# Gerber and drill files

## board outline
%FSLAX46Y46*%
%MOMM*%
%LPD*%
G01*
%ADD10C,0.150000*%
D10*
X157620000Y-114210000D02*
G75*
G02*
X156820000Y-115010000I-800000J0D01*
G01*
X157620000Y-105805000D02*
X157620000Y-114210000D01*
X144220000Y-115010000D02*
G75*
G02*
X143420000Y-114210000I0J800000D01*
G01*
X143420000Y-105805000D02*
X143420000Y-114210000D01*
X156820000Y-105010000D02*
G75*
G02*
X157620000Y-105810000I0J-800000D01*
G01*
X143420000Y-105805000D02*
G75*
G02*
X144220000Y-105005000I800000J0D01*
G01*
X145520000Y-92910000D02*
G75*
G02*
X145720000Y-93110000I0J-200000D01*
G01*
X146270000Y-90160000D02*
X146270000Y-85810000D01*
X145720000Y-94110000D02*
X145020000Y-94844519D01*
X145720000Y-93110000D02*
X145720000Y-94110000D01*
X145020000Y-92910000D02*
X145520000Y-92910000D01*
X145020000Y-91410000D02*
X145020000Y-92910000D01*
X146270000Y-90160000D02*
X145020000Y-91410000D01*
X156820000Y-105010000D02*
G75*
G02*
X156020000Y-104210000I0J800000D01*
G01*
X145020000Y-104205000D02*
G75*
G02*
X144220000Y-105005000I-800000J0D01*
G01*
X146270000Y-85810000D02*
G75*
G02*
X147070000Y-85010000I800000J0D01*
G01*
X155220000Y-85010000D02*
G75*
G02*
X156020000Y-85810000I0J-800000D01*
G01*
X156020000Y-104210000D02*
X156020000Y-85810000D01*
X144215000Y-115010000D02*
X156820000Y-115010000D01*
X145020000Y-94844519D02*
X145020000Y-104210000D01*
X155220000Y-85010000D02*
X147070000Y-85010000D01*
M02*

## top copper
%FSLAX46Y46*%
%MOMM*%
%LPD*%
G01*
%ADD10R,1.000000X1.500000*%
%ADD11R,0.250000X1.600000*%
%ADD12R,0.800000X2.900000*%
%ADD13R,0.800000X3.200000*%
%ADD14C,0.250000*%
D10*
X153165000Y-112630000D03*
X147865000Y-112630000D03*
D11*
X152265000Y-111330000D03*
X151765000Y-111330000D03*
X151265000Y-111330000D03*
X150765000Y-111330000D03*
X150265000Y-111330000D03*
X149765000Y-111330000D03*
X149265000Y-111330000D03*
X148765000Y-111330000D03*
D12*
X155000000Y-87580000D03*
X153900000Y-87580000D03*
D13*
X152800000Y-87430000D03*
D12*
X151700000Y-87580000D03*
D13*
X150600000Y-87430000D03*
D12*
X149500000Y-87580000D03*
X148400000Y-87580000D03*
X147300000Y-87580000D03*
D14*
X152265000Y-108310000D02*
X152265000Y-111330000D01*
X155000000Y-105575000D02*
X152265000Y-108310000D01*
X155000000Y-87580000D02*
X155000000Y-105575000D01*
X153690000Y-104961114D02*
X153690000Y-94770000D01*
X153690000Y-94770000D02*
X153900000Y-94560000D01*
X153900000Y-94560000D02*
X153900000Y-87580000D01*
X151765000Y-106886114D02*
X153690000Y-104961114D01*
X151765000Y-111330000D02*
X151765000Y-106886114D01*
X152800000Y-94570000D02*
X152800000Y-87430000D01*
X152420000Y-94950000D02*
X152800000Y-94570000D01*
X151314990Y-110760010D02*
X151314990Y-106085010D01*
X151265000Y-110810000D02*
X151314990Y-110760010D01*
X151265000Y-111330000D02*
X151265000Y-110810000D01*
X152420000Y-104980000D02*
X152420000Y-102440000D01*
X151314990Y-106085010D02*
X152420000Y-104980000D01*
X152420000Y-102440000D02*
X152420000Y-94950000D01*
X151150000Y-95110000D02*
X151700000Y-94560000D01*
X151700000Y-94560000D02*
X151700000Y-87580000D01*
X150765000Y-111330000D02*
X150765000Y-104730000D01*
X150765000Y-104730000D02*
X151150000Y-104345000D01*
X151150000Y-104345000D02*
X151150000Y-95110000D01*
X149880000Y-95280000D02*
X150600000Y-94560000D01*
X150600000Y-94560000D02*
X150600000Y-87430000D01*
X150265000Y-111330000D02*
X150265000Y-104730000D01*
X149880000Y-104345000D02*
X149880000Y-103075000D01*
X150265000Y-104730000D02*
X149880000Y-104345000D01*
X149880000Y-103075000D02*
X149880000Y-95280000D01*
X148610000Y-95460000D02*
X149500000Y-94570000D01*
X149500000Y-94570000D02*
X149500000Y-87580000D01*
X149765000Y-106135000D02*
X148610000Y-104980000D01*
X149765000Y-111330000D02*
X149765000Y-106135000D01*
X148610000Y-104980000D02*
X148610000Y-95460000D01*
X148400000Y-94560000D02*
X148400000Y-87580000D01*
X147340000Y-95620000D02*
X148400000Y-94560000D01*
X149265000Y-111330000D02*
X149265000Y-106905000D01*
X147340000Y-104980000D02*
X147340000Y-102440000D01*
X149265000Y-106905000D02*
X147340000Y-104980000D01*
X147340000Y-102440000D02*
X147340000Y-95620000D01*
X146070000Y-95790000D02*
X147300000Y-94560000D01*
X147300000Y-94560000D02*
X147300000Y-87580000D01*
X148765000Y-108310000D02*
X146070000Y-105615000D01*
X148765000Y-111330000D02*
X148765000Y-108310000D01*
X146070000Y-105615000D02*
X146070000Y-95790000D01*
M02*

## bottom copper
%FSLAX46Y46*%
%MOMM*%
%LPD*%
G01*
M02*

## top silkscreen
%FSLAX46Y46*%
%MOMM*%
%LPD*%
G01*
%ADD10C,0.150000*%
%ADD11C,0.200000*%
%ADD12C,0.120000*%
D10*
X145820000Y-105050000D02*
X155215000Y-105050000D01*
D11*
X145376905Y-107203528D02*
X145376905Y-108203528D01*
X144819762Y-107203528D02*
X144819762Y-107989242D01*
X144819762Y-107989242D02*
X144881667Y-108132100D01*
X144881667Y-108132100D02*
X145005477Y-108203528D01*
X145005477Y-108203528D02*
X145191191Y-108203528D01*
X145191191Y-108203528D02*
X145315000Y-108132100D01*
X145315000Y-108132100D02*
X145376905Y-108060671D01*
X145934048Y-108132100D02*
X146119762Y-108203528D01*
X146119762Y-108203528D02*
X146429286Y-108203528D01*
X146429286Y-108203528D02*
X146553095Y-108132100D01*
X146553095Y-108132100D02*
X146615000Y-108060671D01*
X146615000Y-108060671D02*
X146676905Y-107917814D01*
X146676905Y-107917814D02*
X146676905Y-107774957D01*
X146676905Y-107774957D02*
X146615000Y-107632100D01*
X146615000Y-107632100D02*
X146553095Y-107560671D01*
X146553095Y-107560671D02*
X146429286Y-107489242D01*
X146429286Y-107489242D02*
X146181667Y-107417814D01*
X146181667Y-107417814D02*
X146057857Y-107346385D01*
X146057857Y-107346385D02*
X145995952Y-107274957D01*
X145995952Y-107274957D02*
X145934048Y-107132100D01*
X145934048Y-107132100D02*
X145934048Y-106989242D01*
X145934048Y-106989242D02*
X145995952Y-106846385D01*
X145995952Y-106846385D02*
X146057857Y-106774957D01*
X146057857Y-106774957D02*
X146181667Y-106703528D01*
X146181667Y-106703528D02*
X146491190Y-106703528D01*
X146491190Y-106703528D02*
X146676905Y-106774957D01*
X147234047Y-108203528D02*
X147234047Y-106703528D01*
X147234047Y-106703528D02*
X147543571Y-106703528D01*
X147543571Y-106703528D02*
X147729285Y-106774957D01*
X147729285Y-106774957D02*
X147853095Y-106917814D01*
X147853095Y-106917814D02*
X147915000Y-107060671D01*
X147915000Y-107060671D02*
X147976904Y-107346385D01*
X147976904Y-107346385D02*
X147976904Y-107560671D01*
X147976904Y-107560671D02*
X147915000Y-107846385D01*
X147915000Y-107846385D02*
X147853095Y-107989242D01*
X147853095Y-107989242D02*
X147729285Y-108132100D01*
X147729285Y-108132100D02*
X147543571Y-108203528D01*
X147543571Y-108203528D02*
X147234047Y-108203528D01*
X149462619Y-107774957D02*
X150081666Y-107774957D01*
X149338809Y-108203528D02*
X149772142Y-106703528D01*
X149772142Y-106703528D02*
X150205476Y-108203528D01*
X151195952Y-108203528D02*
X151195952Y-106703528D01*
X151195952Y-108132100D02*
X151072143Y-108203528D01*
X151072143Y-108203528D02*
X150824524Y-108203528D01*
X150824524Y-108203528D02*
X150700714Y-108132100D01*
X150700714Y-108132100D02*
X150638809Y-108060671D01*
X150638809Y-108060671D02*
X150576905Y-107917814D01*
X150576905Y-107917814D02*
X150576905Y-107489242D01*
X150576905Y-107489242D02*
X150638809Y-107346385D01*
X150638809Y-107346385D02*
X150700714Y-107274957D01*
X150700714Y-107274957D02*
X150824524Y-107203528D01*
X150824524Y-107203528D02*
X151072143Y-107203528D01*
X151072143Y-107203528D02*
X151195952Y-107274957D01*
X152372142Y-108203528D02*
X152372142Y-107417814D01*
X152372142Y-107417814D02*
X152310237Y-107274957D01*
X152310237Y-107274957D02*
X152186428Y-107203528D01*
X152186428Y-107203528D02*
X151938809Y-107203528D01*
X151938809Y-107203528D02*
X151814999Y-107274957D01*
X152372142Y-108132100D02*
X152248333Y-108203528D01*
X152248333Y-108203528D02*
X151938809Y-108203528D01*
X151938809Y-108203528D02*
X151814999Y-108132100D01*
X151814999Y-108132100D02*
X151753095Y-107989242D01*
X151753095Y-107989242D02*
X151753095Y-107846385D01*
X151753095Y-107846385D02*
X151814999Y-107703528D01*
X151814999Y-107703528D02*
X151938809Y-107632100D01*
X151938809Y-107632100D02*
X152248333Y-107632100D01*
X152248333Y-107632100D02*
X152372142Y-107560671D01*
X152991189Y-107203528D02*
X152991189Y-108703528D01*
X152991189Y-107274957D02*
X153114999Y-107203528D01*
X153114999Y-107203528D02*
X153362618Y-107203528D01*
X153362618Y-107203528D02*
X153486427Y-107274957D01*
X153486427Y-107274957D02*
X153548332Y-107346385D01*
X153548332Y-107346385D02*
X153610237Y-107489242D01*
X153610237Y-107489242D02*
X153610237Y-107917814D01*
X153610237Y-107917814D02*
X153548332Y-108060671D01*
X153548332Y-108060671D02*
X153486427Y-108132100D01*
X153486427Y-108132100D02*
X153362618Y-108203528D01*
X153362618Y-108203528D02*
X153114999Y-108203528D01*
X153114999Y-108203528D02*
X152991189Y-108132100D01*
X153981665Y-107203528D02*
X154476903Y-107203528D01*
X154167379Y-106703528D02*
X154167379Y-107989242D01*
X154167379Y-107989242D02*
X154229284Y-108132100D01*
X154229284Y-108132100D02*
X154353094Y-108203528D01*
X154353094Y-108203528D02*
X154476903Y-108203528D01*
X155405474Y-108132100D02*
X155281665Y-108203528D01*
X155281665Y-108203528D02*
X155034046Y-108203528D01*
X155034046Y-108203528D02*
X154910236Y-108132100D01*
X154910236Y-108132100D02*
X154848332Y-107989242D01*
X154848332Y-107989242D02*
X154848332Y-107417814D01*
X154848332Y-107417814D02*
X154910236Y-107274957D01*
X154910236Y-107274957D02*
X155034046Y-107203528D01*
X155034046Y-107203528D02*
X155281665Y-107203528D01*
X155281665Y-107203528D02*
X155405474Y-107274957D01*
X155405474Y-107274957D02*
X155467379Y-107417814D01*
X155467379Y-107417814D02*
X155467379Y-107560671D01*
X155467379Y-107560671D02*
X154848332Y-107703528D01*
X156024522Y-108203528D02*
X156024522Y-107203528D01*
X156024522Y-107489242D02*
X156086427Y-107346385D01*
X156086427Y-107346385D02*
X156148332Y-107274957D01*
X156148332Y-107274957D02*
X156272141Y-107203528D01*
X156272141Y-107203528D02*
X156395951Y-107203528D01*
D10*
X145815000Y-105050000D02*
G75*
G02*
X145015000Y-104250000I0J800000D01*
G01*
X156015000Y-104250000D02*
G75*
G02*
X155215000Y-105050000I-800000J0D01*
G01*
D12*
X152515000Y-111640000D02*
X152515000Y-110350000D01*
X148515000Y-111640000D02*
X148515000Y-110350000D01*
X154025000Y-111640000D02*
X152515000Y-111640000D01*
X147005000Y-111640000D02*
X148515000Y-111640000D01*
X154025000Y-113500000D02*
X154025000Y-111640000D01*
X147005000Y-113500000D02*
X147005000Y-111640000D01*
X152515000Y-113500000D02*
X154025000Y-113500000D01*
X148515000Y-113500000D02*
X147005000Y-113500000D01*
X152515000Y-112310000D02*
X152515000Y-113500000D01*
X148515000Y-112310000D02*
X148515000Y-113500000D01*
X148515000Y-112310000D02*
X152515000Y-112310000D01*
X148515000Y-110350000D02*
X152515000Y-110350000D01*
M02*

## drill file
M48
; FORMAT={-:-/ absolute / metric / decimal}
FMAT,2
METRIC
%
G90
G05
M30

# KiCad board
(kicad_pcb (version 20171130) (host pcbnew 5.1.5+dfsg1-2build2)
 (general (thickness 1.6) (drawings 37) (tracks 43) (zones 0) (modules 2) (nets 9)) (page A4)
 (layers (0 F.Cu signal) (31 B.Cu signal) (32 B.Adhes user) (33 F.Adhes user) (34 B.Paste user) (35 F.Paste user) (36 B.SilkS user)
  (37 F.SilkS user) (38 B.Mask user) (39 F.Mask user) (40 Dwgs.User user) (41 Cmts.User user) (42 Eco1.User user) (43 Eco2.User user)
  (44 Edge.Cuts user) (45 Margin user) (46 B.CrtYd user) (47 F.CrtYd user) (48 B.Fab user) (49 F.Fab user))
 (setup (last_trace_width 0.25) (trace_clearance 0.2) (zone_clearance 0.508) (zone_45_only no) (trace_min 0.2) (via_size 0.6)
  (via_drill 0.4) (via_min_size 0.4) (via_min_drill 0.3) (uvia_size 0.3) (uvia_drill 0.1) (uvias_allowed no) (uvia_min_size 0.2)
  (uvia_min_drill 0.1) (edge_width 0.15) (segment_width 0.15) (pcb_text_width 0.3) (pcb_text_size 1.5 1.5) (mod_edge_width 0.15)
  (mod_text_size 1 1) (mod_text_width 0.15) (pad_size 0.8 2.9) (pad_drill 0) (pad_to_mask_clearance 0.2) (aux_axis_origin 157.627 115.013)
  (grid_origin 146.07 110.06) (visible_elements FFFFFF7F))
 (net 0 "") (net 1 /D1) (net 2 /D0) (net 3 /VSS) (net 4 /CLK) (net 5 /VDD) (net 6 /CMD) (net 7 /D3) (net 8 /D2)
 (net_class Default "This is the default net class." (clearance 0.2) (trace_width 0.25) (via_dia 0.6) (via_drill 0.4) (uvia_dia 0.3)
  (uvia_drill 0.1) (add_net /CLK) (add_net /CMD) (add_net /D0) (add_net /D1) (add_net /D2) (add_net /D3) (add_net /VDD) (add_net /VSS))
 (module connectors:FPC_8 (layer F.Cu) (at 150.515 111.33)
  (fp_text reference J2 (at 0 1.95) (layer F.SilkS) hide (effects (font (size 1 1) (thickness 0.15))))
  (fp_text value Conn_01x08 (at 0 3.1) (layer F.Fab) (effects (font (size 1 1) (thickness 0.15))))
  (fp_line (start 2 0.31) (end 2 -0.98) (layer F.SilkS) (width 0.12))
  (fp_line (start -2 0.31) (end -2 -0.98) (layer F.SilkS) (width 0.12))
  (fp_line (start 3.51 0.31) (end 2 0.31) (layer F.SilkS) (width 0.12))
  (fp_line (start -3.51 0.31) (end -2 0.31) (layer F.SilkS) (width 0.12))
  (fp_line (start 3.51 2.17) (end 3.51 0.31) (layer F.SilkS) (width 0.12))
  (fp_line (start -3.51 2.17) (end -3.51 0.31) (layer F.SilkS) (width 0.12))
  (fp_line (start 2 2.17) (end 3.51 2.17) (layer F.SilkS) (width 0.12))
  (fp_line (start -2 2.17) (end -3.51 2.17) (layer F.SilkS) (width 0.12))
  (fp_line (start 2 0.98) (end 2 2.17) (layer F.SilkS) (width 0.12))
  (fp_line (start -2 0.98) (end -2 2.17) (layer F.SilkS) (width 0.12))
  (fp_line (start -2 0.98) (end 2 0.98) (layer F.SilkS) (width 0.12))
  (fp_line (start -2 -0.98) (end 2 -0.98) (layer F.SilkS) (width 0.12))
  (pad 0 smd rect (at 2.65 1.3) (size 1 1.5) (layers F.Cu F.Paste F.Mask))
  (pad 0 smd rect (at -2.65 1.3) (size 1 1.5) (layers F.Cu F.Paste F.Mask))
  (pad 8 smd rect (at 1.75 0) (size 0.25 1.6) (layers F.Cu F.Paste F.Mask) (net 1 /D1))
  (pad 7 smd rect (at 1.25 0) (size 0.25 1.6) (layers F.Cu F.Paste F.Mask) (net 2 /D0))
  (pad 6 smd rect (at 0.75 0) (size 0.25 1.6) (layers F.Cu F.Paste F.Mask) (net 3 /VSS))
  (pad 5 smd rect (at 0.25 0) (size 0.25 1.6) (layers F.Cu F.Paste F.Mask) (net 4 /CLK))
  (pad 4 smd rect (at -0.25 0) (size 0.25 1.6) (layers F.Cu F.Paste F.Mask) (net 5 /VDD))
  (pad 3 smd rect (at -0.75 0) (size 0.25 1.6) (layers F.Cu F.Paste F.Mask) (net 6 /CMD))
  (pad 2 smd rect (at -1.25 0) (size 0.25 1.6) (layers F.Cu F.Paste F.Mask) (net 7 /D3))
  (pad 1 smd rect (at -1.75 0) (size 0.25 1.6) (layers F.Cu F.Paste F.Mask) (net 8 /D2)))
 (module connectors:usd (layer F.Cu) (at 147.3 87.58)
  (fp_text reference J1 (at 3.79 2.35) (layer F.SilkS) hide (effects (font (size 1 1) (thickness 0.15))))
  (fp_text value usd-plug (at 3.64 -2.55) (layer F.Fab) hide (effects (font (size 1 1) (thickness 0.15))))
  (pad 8 smd rect (at 7.7 0) (size 0.8 2.9) (layers F.Cu F.Paste F.Mask) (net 1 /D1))
  (pad 7 smd rect (at 6.6 0) (size 0.8 2.9) (layers F.Cu F.Paste F.Mask) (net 2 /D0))
  (pad 6 smd rect (at 5.5 -0.15) (size 0.8 3.2) (layers F.Cu F.Paste F.Mask) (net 3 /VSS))
  (pad 5 smd rect (at 4.4 0) (size 0.8 2.9) (layers F.Cu F.Paste F.Mask) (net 4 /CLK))
  (pad 4 smd rect (at 3.3 -0.15) (size 0.8 3.2) (layers F.Cu F.Paste F.Mask) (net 5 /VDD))
  (pad 3 smd rect (at 2.2 0) (size 0.8 2.9) (layers F.Cu F.Paste F.Mask) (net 6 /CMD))
  (pad 2 smd rect (at 1.1 0) (size 0.8 2.9) (layers F.Cu F.Paste F.Mask) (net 7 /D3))
  (pad 1 smd rect (at 0 0) (size 0.8 2.9) (layers F.Cu F.Paste F.Mask) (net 8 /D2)))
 (gr_line (start 145.82 105.05) (end 155.215 105.05) (angle 90) (layer F.SilkS) (width 0.15))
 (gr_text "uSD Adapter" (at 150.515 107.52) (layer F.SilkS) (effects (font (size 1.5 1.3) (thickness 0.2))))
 (gr_arc (start 145.815 104.25) (end 145.815 105.05) (angle 90) (layer F.SilkS) (width 0.15))
 (gr_arc (start 155.215 104.25) (end 156.015 104.25) (angle 90) (layer F.SilkS) (width 0.15))
 (gr_arc (start 156.82 114.21) (end 157.62 114.21) (angle 90) (layer Edge.Cuts) (width 0.15))
 (gr_line (start 157.62 105.805) (end 157.62 114.21) (angle 90) (layer Edge.Cuts) (width 0.15))
 (gr_arc (start 144.22 114.21) (end 144.22 115.01) (angle 90) (layer Edge.Cuts) (width 0.15))
 (gr_line (start 143.42 105.805) (end 143.42 114.21) (angle 90) (layer Edge.Cuts) (width 0.15))
 (gr_arc (start 156.82 105.81) (end 156.82 105.01) (angle 90) (layer Edge.Cuts) (width 0.15))
 (gr_arc (start 144.22 105.805) (end 143.42 105.805) (angle 90) (layer Edge.Cuts) (width 0.15))
 (gr_arc (start 145.52 93.11) (end 145.72 93.11) (angle -90) (layer Edge.Cuts) (width 0.15))
 (gr_line (start 146.27 90.16) (end 146.27 85.81) (angle 90) (layer Edge.Cuts) (width 0.15))
 (gr_line (start 145.72 94.11) (end 145.02 94.844519) (angle 90) (layer Edge.Cuts) (width 0.15))
 (gr_line (start 145.72 93.11) (end 145.72 94.11) (angle 90) (layer Edge.Cuts) (width 0.15))
 (gr_line (start 145.02 92.91) (end 145.52 92.91) (angle 90) (layer Edge.Cuts) (width 0.15))
 (gr_line (start 145.02 91.41) (end 145.02 92.91) (angle 90) (layer Edge.Cuts) (width 0.15))
 (gr_line (start 146.27 90.16) (end 145.02 91.41) (angle 90) (layer Edge.Cuts) (width 0.15))
 (gr_arc (start 156.82 104.21) (end 156.82 105.01) (angle 90) (layer Edge.Cuts) (width 0.15))
 (gr_arc (start 144.22 104.205) (end 145.02 104.205) (angle 90) (layer Edge.Cuts) (width 0.15))
 (gr_arc (start 147.07 85.81) (end 147.07 85.01) (angle -90) (layer Edge.Cuts) (width 0.15))
 (gr_arc (start 155.22 85.81) (end 156.02 85.81) (angle -90) (layer Edge.Cuts) (width 0.15))
 (gr_line (start 156.02 104.21) (end 156.02 85.81) (angle 90) (layer Edge.Cuts) (width 0.15))
 (gr_line (start 144.215 115.01) (end 156.82 115.01) (angle 90) (layer Edge.Cuts) (width 0.15))
 (gr_line (start 145.02 94.844519) (end 145.02 104.21) (angle 90) (layer Edge.Cuts) (width 0.15))
 (gr_line (start 155.22 85.01) (end 147.07 85.01) (angle 90) (layer Edge.Cuts) (width 0.15))
 (segment (start 152.265 108.31) (end 152.265 111.33) (width 0.25) (layer F.Cu) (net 1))
 (segment (start 155 105.575) (end 152.265 108.31) (width 0.25) (layer F.Cu) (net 1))
 (segment (start 155 87.58) (end 155 105.575) (width 0.25) (layer F.Cu) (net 1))
 (segment (start 153.69 104.961114) (end 153.69 94.77) (width 0.25) (layer F.Cu) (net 2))
 (segment (start 153.69 94.77) (end 153.9 94.56) (width 0.25) (layer F.Cu) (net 2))
 (segment (start 153.9 94.56) (end 153.9 87.58) (width 0.25) (layer F.Cu) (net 2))
 (segment (start 151.765 106.886114) (end 153.69 104.961114) (width 0.25) (layer F.Cu) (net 2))
 (segment (start 151.765 111.33) (end 151.765 106.886114) (width 0.25) (layer F.Cu) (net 2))
 (segment (start 152.8 94.57) (end 152.8 87.43) (width 0.25) (layer F.Cu) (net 3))
 (segment (start 152.42 94.95) (end 152.8 94.57) (width 0.25) (layer F.Cu) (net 3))
 (segment (start 151.31499 110.76001) (end 151.31499 106.08501) (width 0.25) (layer F.Cu) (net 3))
 (segment (start 151.265 110.81) (end 151.31499 110.76001) (width 0.25) (layer F.Cu) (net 3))
 (segment (start 151.265 111.33) (end 151.265 110.81) (width 0.25) (layer F.Cu) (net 3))
 (segment (start 152.42 104.98) (end 152.42 102.44) (width 0.25) (layer F.Cu) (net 3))
 (segment (start 151.31499 106.08501) (end 152.42 104.98) (width 0.25) (layer F.Cu) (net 3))
 (segment (start 152.42 102.44) (end 152.42 94.95) (width 0.25) (layer F.Cu) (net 3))
 (segment (start 151.15 95.11) (end 151.7 94.56) (width 0.25) (layer F.Cu) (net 4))
 (segment (start 151.7 94.56) (end 151.7 87.58) (width 0.25) (layer F.Cu) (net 4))
 (segment (start 150.765 111.33) (end 150.765 104.73) (width 0.25) (layer F.Cu) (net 4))
 (segment (start 150.765 104.73) (end 151.15 104.345) (width 0.25) (layer F.Cu) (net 4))
 (segment (start 151.15 104.345) (end 151.15 95.11) (width 0.25) (layer F.Cu) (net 4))
 (segment (start 149.88 95.28) (end 150.6 94.56) (width 0.25) (layer F.Cu) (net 5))
 (segment (start 150.6 94.56) (end 150.6 87.43) (width 0.25) (layer F.Cu) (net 5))
 (segment (start 150.265 111.33) (end 150.265 104.73) (width 0.25) (layer F.Cu) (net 5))
 (segment (start 149.88 104.345) (end 149.88 103.075) (width 0.25) (layer F.Cu) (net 5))
 (segment (start 150.265 104.73) (end 149.88 104.345) (width 0.25) (layer F.Cu) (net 5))
 (segment (start 149.88 103.075) (end 149.88 95.28) (width 0.25) (layer F.Cu) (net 5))
 (segment (start 148.61 95.46) (end 149.5 94.57) (width 0.25) (layer F.Cu) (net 6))
 (segment (start 149.5 94.57) (end 149.5 87.58) (width 0.25) (layer F.Cu) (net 6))
 (segment (start 149.765 106.135) (end 148.61 104.98) (width 0.25) (layer F.Cu) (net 6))
 (segment (start 149.765 111.33) (end 149.765 106.135) (width 0.25) (layer F.Cu) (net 6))
 (segment (start 148.61 104.98) (end 148.61 95.46) (width 0.25) (layer F.Cu) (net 6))
 (segment (start 148.4 94.56) (end 148.4 87.58) (width 0.25) (layer F.Cu) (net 7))
 (segment (start 147.34 95.62) (end 148.4 94.56) (width 0.25) (layer F.Cu) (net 7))
 (segment (start 149.265 111.33) (end 149.265 106.905) (width 0.25) (layer F.Cu) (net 7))
 (segment (start 147.34 104.98) (end 147.34 102.44) (width 0.25) (layer F.Cu) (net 7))
 (segment (start 149.265 106.905) (end 147.34 104.98) (width 0.25) (layer F.Cu) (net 7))
 (segment (start 147.34 102.44) (end 147.34 95.62) (width 0.25) (layer F.Cu) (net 7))
 (segment (start 146.07 95.79) (end 147.3 94.56) (width 0.25) (layer F.Cu) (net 8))
 (segment (start 147.3 94.56) (end 147.3 87.58) (width 0.25) (layer F.Cu) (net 8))
 (segment (start 148.765 108.31) (end 146.07 105.615) (width 0.25) (layer F.Cu) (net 8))
 (segment (start 148.765 111.33) (end 148.765 108.31) (width 0.25) (layer F.Cu) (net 8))
 (segment (start 146.07 105.615) (end 146.07 95.79) (width 0.25) (layer F.Cu) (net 8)))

